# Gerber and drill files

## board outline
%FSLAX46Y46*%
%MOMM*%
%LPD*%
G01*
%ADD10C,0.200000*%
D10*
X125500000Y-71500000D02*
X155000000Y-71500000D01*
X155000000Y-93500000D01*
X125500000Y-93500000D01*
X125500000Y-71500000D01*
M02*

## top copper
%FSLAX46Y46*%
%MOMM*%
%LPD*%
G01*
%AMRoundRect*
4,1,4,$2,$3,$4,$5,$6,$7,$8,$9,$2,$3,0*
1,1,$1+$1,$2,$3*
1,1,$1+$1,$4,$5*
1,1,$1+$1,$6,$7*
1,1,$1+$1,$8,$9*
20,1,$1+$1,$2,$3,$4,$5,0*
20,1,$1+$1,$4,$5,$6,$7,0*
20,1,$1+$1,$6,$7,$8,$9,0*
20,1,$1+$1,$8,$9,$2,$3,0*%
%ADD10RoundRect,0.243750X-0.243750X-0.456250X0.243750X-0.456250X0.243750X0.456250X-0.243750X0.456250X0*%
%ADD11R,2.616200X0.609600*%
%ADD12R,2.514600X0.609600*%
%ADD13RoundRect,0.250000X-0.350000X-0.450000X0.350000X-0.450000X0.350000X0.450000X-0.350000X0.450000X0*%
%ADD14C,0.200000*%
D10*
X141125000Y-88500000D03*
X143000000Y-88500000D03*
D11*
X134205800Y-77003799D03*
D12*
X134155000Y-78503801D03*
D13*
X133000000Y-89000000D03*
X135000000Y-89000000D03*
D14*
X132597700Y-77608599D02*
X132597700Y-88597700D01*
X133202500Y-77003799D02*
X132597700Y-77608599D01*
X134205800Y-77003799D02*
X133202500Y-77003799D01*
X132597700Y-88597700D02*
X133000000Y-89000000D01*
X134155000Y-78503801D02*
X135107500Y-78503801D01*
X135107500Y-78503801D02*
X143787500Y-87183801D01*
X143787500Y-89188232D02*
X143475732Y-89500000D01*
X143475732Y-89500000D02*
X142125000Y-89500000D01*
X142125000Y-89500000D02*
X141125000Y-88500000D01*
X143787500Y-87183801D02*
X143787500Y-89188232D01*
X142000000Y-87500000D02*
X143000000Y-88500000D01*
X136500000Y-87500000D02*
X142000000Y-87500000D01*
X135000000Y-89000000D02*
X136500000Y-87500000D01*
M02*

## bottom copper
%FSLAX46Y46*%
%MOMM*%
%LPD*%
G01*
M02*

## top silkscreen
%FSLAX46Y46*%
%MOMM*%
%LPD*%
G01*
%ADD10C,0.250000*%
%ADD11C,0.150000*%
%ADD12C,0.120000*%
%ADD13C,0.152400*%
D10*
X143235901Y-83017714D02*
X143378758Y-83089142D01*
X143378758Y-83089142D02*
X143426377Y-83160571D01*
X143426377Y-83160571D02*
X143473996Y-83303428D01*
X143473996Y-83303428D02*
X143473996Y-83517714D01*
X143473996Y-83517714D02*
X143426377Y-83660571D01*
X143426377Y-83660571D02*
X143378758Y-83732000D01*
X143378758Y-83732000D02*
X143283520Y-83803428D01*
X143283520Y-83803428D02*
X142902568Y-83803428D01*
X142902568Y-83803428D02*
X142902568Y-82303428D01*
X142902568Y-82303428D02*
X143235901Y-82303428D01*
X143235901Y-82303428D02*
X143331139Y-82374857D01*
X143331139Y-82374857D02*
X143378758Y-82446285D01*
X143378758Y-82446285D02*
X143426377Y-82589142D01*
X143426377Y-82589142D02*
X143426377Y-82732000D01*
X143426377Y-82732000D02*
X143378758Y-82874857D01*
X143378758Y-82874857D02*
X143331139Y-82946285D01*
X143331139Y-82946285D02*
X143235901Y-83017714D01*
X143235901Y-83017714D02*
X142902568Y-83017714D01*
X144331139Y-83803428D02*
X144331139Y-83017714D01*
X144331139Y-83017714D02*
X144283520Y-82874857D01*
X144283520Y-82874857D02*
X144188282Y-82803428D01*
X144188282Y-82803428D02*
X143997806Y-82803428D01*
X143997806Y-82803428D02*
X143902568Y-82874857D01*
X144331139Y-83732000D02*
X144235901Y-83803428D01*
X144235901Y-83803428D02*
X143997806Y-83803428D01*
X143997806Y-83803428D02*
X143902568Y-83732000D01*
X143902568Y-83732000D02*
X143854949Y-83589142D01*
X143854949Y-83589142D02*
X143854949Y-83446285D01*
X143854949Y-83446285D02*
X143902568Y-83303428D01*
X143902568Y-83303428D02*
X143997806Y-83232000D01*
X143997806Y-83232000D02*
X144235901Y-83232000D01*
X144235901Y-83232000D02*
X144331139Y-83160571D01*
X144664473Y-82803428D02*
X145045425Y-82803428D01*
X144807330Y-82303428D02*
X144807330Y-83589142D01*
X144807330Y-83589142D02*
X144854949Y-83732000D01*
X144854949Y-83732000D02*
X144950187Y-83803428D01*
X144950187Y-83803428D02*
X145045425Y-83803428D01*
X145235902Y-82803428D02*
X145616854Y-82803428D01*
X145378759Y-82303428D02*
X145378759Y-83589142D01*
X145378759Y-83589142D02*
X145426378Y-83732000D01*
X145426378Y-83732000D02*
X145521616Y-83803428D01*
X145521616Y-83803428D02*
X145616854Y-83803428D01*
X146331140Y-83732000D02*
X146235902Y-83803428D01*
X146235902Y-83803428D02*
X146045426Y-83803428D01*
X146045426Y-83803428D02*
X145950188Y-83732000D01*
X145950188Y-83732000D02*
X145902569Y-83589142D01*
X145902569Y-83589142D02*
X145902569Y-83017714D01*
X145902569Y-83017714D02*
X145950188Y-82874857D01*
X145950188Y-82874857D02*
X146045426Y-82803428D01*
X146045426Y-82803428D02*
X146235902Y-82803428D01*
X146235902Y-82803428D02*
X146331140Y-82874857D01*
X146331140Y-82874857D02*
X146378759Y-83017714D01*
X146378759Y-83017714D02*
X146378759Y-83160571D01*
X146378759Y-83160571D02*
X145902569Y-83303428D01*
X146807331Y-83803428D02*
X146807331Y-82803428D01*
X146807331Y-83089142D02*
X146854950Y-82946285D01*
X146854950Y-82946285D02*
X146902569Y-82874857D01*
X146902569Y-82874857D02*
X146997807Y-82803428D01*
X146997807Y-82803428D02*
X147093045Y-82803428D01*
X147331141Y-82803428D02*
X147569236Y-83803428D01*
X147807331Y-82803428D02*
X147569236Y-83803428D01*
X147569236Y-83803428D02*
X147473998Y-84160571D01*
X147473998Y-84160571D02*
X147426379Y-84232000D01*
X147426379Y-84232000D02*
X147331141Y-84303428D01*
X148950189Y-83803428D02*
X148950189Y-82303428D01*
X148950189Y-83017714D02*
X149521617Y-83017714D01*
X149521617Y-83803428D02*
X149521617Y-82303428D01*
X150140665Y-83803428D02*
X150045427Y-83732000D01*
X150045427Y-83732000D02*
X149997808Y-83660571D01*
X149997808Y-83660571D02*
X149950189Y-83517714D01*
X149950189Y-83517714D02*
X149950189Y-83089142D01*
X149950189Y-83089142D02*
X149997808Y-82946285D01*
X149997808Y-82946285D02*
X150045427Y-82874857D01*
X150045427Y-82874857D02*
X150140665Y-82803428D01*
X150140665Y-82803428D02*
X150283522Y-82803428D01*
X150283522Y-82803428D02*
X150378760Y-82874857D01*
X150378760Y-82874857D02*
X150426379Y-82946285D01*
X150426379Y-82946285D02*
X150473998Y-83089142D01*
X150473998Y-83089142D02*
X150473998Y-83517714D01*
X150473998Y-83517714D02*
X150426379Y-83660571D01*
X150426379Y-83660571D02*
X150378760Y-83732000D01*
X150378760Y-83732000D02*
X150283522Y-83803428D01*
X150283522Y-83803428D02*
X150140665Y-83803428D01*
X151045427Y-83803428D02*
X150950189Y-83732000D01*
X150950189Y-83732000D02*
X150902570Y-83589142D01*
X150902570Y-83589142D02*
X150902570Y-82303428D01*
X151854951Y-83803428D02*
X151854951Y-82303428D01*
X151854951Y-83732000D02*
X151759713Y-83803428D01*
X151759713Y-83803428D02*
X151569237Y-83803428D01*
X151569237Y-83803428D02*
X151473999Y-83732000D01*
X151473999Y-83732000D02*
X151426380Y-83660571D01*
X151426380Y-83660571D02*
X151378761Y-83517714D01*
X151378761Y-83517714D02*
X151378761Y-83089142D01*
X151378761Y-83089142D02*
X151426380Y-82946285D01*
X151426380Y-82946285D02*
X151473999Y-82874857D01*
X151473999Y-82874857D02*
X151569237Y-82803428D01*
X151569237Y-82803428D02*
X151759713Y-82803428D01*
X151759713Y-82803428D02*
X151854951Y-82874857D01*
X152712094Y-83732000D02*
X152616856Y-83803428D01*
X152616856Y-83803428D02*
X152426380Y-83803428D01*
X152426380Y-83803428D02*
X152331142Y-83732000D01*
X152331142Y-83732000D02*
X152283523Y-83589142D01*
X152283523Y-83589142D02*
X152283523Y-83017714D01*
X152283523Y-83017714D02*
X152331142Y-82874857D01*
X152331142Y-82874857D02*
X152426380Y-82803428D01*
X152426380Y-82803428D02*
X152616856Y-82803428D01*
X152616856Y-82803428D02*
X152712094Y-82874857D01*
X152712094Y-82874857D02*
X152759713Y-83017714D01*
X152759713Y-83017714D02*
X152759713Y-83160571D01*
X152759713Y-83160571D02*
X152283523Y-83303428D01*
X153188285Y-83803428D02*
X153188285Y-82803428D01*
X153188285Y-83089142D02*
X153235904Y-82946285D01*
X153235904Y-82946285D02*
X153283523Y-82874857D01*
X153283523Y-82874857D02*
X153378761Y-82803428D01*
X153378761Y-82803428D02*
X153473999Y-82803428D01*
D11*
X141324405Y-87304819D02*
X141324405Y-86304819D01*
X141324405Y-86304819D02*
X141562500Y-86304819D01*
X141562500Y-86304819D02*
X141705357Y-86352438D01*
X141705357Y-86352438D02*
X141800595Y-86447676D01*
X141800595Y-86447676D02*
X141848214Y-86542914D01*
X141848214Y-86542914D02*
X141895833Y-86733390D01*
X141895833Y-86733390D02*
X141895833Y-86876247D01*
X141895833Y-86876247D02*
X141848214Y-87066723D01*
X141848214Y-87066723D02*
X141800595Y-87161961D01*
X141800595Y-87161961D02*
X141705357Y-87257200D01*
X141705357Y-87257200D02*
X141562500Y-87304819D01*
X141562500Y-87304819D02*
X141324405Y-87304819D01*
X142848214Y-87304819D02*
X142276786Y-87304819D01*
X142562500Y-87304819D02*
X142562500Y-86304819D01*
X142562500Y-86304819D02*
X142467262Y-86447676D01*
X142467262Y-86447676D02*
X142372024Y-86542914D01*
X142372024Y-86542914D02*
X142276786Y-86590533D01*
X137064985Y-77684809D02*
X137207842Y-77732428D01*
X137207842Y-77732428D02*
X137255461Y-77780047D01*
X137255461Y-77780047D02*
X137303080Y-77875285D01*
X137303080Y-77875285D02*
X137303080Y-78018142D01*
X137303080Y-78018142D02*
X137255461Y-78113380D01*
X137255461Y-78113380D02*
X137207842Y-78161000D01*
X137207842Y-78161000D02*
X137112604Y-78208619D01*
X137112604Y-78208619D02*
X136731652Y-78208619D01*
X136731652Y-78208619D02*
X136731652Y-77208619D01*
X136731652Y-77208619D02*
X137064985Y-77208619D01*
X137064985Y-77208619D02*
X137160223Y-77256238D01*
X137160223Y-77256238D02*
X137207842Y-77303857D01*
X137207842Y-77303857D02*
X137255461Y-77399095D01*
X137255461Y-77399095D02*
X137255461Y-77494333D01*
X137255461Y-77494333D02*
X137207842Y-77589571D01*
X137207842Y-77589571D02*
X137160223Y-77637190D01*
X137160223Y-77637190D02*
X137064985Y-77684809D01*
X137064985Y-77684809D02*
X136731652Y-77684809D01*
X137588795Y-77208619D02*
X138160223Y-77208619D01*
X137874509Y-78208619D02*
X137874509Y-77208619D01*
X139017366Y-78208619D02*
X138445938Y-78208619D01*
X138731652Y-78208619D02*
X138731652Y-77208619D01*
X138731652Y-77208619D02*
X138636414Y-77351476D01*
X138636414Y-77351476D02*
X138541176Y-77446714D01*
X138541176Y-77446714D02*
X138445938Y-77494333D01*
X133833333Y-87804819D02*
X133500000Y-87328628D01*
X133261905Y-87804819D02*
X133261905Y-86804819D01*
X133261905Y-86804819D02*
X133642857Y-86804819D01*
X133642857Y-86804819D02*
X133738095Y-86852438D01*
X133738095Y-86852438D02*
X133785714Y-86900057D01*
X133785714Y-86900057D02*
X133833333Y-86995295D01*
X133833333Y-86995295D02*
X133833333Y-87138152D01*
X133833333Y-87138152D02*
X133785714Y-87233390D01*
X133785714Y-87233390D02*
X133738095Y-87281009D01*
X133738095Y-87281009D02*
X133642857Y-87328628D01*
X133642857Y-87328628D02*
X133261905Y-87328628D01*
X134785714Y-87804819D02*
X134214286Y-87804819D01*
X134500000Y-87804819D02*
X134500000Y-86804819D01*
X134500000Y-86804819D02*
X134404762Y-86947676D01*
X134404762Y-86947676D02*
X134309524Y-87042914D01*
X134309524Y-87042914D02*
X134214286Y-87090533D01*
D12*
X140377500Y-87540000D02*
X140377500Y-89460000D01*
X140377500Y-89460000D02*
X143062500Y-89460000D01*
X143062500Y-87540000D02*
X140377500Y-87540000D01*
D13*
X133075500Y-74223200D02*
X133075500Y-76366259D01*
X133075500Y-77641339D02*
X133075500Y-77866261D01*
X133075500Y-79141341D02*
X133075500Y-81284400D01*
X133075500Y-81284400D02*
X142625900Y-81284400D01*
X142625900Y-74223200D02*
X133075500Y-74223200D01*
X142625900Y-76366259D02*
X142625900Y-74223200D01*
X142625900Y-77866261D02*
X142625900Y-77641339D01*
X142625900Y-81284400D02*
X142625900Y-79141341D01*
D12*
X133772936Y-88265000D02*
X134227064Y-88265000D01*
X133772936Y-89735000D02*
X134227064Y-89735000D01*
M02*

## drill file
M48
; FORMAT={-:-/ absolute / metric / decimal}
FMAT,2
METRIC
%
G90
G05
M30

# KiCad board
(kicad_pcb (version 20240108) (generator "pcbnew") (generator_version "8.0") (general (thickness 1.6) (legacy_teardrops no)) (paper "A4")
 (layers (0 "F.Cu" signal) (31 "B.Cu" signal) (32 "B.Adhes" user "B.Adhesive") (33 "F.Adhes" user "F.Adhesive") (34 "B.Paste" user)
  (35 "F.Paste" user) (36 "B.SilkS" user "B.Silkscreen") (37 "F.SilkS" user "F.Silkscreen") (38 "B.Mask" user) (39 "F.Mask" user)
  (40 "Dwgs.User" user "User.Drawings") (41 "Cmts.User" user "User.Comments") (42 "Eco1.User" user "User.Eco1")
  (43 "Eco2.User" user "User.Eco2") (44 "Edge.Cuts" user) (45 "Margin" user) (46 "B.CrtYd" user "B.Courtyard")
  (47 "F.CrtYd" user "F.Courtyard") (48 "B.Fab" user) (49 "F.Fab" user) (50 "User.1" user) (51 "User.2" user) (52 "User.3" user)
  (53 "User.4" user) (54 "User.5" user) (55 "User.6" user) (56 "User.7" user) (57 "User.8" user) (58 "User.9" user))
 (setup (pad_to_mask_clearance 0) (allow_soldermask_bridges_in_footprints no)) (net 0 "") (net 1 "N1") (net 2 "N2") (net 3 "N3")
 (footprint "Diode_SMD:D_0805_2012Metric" (layer "F.Cu") (at 142.0625 88.5)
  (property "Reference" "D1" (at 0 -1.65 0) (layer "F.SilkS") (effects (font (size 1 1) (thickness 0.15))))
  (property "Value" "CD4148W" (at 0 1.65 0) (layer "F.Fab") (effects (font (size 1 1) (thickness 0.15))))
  (fp_line (start -1.685 -0.96) (end -1.685 0.96) (stroke (width 0.12) (type solid)) (layer "F.SilkS"))
  (fp_line (start -1.685 0.96) (end 1 0.96) (stroke (width 0.12) (type solid)) (layer "F.SilkS"))
  (fp_line (start 1 -0.96) (end -1.685 -0.96) (stroke (width 0.12) (type solid)) (layer "F.SilkS"))
  (pad "1" smd roundrect (at -0.9375 0) (size 0.975 1.4) (layers "F.Cu" "F.Paste" "F.Mask") (roundrect_rratio 0.25) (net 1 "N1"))
  (pad "2" smd roundrect (at 0.9375 0) (size 0.975 1.4) (layers "F.Cu" "F.Paste" "F.Mask") (roundrect_rratio 0.25) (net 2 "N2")))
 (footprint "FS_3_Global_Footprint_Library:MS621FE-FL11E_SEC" (layer "F.Cu") (at 137.8507 77.7538)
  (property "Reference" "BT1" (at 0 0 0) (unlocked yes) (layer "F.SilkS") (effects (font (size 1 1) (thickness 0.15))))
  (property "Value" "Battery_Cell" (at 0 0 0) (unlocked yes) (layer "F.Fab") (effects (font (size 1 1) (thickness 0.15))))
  (fp_line (start -4.7752 -3.5306) (end -4.7752 -1.387541) (stroke (width 0.1524) (type solid)) (layer "F.SilkS"))
  (fp_line (start -4.7752 -0.112461) (end -4.7752 0.112461) (stroke (width 0.1524) (type solid)) (layer "F.SilkS"))
  (fp_line (start -4.7752 1.387541) (end -4.7752 3.5306) (stroke (width 0.1524) (type solid)) (layer "F.SilkS"))
  (fp_line (start -4.7752 3.5306) (end 4.7752 3.5306) (stroke (width 0.1524) (type solid)) (layer "F.SilkS"))
  (fp_line (start 4.7752 -3.5306) (end -4.7752 -3.5306) (stroke (width 0.1524) (type solid)) (layer "F.SilkS"))
  (fp_line (start 4.7752 -1.387541) (end 4.7752 -3.5306) (stroke (width 0.1524) (type solid)) (layer "F.SilkS"))
  (fp_line (start 4.7752 0.112461) (end 4.7752 -0.112461) (stroke (width 0.1524) (type solid)) (layer "F.SilkS"))
  (fp_line (start 4.7752 3.5306) (end 4.7752 1.387541) (stroke (width 0.1524) (type solid)) (layer "F.SilkS"))
  (pad "1" smd rect (at -3.6449 -0.750001) (size 2.6162 0.6096) (layers "F.Cu" "F.Paste" "F.Mask") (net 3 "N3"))
  (pad "2" smd rect (at -3.6957 0.750001) (size 2.5146 0.6096) (layers "F.Cu" "F.Paste" "F.Mask") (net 1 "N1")))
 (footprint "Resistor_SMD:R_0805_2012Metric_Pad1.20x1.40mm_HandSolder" (layer "F.Cu") (at 134 89)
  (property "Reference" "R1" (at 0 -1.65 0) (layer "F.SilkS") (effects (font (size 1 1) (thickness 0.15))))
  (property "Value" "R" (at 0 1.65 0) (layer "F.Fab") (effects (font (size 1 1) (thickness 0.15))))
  (fp_line (start -0.227064 -0.735) (end 0.227064 -0.735) (stroke (width 0.12) (type solid)) (layer "F.SilkS"))
  (fp_line (start -0.227064 0.735) (end 0.227064 0.735) (stroke (width 0.12) (type solid)) (layer "F.SilkS"))
  (pad "1" smd roundrect (at -1 0) (size 1.2 1.4) (layers "F.Cu" "F.Paste" "F.Mask") (roundrect_rratio 0.208333) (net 3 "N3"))
  (pad "2" smd roundrect (at 1 0) (size 1.2 1.4) (layers "F.Cu" "F.Paste" "F.Mask") (roundrect_rratio 0.208333) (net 2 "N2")))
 (gr_rect (start 125.5 71.5) (end 155 93.5) (stroke (width 0.2) (type default)) (fill none) (layer "Edge.Cuts"))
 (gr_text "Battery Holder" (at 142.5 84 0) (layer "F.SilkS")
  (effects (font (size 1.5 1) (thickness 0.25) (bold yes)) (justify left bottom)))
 (segment (start 132.5977 77.608599) (end 132.5977 88.5977) (width 0.2) (layer "F.Cu") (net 3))
 (segment (start 133.2025 77.003799) (end 132.5977 77.608599) (width 0.2) (layer "F.Cu") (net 3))
 (segment (start 134.2058 77.003799) (end 133.2025 77.003799) (width 0.2) (layer "F.Cu") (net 3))
 (segment (start 132.5977 88.5977) (end 133 89) (width 0.2) (layer "F.Cu") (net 3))
 (segment (start 134.155 78.503801) (end 135.1075 78.503801) (width 0.2) (layer "F.Cu") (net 1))
 (segment (start 135.1075 78.503801) (end 143.7875 87.183801) (width 0.2) (layer "F.Cu") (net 1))
 (segment (start 143.7875 89.188232) (end 143.475732 89.5) (width 0.2) (layer "F.Cu") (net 1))
 (segment (start 143.475732 89.5) (end 142.125 89.5) (width 0.2) (layer "F.Cu") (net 1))
 (segment (start 142.125 89.5) (end 141.125 88.5) (width 0.2) (layer "F.Cu") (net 1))
 (segment (start 143.7875 87.183801) (end 143.7875 89.188232) (width 0.2) (layer "F.Cu") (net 1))
 (segment (start 142 87.5) (end 143 88.5) (width 0.2) (layer "F.Cu") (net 2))
 (segment (start 136.5 87.5) (end 142 87.5) (width 0.2) (layer "F.Cu") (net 2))
 (segment (start 135 89) (end 136.5 87.5) (width 0.2) (layer "F.Cu") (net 2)))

